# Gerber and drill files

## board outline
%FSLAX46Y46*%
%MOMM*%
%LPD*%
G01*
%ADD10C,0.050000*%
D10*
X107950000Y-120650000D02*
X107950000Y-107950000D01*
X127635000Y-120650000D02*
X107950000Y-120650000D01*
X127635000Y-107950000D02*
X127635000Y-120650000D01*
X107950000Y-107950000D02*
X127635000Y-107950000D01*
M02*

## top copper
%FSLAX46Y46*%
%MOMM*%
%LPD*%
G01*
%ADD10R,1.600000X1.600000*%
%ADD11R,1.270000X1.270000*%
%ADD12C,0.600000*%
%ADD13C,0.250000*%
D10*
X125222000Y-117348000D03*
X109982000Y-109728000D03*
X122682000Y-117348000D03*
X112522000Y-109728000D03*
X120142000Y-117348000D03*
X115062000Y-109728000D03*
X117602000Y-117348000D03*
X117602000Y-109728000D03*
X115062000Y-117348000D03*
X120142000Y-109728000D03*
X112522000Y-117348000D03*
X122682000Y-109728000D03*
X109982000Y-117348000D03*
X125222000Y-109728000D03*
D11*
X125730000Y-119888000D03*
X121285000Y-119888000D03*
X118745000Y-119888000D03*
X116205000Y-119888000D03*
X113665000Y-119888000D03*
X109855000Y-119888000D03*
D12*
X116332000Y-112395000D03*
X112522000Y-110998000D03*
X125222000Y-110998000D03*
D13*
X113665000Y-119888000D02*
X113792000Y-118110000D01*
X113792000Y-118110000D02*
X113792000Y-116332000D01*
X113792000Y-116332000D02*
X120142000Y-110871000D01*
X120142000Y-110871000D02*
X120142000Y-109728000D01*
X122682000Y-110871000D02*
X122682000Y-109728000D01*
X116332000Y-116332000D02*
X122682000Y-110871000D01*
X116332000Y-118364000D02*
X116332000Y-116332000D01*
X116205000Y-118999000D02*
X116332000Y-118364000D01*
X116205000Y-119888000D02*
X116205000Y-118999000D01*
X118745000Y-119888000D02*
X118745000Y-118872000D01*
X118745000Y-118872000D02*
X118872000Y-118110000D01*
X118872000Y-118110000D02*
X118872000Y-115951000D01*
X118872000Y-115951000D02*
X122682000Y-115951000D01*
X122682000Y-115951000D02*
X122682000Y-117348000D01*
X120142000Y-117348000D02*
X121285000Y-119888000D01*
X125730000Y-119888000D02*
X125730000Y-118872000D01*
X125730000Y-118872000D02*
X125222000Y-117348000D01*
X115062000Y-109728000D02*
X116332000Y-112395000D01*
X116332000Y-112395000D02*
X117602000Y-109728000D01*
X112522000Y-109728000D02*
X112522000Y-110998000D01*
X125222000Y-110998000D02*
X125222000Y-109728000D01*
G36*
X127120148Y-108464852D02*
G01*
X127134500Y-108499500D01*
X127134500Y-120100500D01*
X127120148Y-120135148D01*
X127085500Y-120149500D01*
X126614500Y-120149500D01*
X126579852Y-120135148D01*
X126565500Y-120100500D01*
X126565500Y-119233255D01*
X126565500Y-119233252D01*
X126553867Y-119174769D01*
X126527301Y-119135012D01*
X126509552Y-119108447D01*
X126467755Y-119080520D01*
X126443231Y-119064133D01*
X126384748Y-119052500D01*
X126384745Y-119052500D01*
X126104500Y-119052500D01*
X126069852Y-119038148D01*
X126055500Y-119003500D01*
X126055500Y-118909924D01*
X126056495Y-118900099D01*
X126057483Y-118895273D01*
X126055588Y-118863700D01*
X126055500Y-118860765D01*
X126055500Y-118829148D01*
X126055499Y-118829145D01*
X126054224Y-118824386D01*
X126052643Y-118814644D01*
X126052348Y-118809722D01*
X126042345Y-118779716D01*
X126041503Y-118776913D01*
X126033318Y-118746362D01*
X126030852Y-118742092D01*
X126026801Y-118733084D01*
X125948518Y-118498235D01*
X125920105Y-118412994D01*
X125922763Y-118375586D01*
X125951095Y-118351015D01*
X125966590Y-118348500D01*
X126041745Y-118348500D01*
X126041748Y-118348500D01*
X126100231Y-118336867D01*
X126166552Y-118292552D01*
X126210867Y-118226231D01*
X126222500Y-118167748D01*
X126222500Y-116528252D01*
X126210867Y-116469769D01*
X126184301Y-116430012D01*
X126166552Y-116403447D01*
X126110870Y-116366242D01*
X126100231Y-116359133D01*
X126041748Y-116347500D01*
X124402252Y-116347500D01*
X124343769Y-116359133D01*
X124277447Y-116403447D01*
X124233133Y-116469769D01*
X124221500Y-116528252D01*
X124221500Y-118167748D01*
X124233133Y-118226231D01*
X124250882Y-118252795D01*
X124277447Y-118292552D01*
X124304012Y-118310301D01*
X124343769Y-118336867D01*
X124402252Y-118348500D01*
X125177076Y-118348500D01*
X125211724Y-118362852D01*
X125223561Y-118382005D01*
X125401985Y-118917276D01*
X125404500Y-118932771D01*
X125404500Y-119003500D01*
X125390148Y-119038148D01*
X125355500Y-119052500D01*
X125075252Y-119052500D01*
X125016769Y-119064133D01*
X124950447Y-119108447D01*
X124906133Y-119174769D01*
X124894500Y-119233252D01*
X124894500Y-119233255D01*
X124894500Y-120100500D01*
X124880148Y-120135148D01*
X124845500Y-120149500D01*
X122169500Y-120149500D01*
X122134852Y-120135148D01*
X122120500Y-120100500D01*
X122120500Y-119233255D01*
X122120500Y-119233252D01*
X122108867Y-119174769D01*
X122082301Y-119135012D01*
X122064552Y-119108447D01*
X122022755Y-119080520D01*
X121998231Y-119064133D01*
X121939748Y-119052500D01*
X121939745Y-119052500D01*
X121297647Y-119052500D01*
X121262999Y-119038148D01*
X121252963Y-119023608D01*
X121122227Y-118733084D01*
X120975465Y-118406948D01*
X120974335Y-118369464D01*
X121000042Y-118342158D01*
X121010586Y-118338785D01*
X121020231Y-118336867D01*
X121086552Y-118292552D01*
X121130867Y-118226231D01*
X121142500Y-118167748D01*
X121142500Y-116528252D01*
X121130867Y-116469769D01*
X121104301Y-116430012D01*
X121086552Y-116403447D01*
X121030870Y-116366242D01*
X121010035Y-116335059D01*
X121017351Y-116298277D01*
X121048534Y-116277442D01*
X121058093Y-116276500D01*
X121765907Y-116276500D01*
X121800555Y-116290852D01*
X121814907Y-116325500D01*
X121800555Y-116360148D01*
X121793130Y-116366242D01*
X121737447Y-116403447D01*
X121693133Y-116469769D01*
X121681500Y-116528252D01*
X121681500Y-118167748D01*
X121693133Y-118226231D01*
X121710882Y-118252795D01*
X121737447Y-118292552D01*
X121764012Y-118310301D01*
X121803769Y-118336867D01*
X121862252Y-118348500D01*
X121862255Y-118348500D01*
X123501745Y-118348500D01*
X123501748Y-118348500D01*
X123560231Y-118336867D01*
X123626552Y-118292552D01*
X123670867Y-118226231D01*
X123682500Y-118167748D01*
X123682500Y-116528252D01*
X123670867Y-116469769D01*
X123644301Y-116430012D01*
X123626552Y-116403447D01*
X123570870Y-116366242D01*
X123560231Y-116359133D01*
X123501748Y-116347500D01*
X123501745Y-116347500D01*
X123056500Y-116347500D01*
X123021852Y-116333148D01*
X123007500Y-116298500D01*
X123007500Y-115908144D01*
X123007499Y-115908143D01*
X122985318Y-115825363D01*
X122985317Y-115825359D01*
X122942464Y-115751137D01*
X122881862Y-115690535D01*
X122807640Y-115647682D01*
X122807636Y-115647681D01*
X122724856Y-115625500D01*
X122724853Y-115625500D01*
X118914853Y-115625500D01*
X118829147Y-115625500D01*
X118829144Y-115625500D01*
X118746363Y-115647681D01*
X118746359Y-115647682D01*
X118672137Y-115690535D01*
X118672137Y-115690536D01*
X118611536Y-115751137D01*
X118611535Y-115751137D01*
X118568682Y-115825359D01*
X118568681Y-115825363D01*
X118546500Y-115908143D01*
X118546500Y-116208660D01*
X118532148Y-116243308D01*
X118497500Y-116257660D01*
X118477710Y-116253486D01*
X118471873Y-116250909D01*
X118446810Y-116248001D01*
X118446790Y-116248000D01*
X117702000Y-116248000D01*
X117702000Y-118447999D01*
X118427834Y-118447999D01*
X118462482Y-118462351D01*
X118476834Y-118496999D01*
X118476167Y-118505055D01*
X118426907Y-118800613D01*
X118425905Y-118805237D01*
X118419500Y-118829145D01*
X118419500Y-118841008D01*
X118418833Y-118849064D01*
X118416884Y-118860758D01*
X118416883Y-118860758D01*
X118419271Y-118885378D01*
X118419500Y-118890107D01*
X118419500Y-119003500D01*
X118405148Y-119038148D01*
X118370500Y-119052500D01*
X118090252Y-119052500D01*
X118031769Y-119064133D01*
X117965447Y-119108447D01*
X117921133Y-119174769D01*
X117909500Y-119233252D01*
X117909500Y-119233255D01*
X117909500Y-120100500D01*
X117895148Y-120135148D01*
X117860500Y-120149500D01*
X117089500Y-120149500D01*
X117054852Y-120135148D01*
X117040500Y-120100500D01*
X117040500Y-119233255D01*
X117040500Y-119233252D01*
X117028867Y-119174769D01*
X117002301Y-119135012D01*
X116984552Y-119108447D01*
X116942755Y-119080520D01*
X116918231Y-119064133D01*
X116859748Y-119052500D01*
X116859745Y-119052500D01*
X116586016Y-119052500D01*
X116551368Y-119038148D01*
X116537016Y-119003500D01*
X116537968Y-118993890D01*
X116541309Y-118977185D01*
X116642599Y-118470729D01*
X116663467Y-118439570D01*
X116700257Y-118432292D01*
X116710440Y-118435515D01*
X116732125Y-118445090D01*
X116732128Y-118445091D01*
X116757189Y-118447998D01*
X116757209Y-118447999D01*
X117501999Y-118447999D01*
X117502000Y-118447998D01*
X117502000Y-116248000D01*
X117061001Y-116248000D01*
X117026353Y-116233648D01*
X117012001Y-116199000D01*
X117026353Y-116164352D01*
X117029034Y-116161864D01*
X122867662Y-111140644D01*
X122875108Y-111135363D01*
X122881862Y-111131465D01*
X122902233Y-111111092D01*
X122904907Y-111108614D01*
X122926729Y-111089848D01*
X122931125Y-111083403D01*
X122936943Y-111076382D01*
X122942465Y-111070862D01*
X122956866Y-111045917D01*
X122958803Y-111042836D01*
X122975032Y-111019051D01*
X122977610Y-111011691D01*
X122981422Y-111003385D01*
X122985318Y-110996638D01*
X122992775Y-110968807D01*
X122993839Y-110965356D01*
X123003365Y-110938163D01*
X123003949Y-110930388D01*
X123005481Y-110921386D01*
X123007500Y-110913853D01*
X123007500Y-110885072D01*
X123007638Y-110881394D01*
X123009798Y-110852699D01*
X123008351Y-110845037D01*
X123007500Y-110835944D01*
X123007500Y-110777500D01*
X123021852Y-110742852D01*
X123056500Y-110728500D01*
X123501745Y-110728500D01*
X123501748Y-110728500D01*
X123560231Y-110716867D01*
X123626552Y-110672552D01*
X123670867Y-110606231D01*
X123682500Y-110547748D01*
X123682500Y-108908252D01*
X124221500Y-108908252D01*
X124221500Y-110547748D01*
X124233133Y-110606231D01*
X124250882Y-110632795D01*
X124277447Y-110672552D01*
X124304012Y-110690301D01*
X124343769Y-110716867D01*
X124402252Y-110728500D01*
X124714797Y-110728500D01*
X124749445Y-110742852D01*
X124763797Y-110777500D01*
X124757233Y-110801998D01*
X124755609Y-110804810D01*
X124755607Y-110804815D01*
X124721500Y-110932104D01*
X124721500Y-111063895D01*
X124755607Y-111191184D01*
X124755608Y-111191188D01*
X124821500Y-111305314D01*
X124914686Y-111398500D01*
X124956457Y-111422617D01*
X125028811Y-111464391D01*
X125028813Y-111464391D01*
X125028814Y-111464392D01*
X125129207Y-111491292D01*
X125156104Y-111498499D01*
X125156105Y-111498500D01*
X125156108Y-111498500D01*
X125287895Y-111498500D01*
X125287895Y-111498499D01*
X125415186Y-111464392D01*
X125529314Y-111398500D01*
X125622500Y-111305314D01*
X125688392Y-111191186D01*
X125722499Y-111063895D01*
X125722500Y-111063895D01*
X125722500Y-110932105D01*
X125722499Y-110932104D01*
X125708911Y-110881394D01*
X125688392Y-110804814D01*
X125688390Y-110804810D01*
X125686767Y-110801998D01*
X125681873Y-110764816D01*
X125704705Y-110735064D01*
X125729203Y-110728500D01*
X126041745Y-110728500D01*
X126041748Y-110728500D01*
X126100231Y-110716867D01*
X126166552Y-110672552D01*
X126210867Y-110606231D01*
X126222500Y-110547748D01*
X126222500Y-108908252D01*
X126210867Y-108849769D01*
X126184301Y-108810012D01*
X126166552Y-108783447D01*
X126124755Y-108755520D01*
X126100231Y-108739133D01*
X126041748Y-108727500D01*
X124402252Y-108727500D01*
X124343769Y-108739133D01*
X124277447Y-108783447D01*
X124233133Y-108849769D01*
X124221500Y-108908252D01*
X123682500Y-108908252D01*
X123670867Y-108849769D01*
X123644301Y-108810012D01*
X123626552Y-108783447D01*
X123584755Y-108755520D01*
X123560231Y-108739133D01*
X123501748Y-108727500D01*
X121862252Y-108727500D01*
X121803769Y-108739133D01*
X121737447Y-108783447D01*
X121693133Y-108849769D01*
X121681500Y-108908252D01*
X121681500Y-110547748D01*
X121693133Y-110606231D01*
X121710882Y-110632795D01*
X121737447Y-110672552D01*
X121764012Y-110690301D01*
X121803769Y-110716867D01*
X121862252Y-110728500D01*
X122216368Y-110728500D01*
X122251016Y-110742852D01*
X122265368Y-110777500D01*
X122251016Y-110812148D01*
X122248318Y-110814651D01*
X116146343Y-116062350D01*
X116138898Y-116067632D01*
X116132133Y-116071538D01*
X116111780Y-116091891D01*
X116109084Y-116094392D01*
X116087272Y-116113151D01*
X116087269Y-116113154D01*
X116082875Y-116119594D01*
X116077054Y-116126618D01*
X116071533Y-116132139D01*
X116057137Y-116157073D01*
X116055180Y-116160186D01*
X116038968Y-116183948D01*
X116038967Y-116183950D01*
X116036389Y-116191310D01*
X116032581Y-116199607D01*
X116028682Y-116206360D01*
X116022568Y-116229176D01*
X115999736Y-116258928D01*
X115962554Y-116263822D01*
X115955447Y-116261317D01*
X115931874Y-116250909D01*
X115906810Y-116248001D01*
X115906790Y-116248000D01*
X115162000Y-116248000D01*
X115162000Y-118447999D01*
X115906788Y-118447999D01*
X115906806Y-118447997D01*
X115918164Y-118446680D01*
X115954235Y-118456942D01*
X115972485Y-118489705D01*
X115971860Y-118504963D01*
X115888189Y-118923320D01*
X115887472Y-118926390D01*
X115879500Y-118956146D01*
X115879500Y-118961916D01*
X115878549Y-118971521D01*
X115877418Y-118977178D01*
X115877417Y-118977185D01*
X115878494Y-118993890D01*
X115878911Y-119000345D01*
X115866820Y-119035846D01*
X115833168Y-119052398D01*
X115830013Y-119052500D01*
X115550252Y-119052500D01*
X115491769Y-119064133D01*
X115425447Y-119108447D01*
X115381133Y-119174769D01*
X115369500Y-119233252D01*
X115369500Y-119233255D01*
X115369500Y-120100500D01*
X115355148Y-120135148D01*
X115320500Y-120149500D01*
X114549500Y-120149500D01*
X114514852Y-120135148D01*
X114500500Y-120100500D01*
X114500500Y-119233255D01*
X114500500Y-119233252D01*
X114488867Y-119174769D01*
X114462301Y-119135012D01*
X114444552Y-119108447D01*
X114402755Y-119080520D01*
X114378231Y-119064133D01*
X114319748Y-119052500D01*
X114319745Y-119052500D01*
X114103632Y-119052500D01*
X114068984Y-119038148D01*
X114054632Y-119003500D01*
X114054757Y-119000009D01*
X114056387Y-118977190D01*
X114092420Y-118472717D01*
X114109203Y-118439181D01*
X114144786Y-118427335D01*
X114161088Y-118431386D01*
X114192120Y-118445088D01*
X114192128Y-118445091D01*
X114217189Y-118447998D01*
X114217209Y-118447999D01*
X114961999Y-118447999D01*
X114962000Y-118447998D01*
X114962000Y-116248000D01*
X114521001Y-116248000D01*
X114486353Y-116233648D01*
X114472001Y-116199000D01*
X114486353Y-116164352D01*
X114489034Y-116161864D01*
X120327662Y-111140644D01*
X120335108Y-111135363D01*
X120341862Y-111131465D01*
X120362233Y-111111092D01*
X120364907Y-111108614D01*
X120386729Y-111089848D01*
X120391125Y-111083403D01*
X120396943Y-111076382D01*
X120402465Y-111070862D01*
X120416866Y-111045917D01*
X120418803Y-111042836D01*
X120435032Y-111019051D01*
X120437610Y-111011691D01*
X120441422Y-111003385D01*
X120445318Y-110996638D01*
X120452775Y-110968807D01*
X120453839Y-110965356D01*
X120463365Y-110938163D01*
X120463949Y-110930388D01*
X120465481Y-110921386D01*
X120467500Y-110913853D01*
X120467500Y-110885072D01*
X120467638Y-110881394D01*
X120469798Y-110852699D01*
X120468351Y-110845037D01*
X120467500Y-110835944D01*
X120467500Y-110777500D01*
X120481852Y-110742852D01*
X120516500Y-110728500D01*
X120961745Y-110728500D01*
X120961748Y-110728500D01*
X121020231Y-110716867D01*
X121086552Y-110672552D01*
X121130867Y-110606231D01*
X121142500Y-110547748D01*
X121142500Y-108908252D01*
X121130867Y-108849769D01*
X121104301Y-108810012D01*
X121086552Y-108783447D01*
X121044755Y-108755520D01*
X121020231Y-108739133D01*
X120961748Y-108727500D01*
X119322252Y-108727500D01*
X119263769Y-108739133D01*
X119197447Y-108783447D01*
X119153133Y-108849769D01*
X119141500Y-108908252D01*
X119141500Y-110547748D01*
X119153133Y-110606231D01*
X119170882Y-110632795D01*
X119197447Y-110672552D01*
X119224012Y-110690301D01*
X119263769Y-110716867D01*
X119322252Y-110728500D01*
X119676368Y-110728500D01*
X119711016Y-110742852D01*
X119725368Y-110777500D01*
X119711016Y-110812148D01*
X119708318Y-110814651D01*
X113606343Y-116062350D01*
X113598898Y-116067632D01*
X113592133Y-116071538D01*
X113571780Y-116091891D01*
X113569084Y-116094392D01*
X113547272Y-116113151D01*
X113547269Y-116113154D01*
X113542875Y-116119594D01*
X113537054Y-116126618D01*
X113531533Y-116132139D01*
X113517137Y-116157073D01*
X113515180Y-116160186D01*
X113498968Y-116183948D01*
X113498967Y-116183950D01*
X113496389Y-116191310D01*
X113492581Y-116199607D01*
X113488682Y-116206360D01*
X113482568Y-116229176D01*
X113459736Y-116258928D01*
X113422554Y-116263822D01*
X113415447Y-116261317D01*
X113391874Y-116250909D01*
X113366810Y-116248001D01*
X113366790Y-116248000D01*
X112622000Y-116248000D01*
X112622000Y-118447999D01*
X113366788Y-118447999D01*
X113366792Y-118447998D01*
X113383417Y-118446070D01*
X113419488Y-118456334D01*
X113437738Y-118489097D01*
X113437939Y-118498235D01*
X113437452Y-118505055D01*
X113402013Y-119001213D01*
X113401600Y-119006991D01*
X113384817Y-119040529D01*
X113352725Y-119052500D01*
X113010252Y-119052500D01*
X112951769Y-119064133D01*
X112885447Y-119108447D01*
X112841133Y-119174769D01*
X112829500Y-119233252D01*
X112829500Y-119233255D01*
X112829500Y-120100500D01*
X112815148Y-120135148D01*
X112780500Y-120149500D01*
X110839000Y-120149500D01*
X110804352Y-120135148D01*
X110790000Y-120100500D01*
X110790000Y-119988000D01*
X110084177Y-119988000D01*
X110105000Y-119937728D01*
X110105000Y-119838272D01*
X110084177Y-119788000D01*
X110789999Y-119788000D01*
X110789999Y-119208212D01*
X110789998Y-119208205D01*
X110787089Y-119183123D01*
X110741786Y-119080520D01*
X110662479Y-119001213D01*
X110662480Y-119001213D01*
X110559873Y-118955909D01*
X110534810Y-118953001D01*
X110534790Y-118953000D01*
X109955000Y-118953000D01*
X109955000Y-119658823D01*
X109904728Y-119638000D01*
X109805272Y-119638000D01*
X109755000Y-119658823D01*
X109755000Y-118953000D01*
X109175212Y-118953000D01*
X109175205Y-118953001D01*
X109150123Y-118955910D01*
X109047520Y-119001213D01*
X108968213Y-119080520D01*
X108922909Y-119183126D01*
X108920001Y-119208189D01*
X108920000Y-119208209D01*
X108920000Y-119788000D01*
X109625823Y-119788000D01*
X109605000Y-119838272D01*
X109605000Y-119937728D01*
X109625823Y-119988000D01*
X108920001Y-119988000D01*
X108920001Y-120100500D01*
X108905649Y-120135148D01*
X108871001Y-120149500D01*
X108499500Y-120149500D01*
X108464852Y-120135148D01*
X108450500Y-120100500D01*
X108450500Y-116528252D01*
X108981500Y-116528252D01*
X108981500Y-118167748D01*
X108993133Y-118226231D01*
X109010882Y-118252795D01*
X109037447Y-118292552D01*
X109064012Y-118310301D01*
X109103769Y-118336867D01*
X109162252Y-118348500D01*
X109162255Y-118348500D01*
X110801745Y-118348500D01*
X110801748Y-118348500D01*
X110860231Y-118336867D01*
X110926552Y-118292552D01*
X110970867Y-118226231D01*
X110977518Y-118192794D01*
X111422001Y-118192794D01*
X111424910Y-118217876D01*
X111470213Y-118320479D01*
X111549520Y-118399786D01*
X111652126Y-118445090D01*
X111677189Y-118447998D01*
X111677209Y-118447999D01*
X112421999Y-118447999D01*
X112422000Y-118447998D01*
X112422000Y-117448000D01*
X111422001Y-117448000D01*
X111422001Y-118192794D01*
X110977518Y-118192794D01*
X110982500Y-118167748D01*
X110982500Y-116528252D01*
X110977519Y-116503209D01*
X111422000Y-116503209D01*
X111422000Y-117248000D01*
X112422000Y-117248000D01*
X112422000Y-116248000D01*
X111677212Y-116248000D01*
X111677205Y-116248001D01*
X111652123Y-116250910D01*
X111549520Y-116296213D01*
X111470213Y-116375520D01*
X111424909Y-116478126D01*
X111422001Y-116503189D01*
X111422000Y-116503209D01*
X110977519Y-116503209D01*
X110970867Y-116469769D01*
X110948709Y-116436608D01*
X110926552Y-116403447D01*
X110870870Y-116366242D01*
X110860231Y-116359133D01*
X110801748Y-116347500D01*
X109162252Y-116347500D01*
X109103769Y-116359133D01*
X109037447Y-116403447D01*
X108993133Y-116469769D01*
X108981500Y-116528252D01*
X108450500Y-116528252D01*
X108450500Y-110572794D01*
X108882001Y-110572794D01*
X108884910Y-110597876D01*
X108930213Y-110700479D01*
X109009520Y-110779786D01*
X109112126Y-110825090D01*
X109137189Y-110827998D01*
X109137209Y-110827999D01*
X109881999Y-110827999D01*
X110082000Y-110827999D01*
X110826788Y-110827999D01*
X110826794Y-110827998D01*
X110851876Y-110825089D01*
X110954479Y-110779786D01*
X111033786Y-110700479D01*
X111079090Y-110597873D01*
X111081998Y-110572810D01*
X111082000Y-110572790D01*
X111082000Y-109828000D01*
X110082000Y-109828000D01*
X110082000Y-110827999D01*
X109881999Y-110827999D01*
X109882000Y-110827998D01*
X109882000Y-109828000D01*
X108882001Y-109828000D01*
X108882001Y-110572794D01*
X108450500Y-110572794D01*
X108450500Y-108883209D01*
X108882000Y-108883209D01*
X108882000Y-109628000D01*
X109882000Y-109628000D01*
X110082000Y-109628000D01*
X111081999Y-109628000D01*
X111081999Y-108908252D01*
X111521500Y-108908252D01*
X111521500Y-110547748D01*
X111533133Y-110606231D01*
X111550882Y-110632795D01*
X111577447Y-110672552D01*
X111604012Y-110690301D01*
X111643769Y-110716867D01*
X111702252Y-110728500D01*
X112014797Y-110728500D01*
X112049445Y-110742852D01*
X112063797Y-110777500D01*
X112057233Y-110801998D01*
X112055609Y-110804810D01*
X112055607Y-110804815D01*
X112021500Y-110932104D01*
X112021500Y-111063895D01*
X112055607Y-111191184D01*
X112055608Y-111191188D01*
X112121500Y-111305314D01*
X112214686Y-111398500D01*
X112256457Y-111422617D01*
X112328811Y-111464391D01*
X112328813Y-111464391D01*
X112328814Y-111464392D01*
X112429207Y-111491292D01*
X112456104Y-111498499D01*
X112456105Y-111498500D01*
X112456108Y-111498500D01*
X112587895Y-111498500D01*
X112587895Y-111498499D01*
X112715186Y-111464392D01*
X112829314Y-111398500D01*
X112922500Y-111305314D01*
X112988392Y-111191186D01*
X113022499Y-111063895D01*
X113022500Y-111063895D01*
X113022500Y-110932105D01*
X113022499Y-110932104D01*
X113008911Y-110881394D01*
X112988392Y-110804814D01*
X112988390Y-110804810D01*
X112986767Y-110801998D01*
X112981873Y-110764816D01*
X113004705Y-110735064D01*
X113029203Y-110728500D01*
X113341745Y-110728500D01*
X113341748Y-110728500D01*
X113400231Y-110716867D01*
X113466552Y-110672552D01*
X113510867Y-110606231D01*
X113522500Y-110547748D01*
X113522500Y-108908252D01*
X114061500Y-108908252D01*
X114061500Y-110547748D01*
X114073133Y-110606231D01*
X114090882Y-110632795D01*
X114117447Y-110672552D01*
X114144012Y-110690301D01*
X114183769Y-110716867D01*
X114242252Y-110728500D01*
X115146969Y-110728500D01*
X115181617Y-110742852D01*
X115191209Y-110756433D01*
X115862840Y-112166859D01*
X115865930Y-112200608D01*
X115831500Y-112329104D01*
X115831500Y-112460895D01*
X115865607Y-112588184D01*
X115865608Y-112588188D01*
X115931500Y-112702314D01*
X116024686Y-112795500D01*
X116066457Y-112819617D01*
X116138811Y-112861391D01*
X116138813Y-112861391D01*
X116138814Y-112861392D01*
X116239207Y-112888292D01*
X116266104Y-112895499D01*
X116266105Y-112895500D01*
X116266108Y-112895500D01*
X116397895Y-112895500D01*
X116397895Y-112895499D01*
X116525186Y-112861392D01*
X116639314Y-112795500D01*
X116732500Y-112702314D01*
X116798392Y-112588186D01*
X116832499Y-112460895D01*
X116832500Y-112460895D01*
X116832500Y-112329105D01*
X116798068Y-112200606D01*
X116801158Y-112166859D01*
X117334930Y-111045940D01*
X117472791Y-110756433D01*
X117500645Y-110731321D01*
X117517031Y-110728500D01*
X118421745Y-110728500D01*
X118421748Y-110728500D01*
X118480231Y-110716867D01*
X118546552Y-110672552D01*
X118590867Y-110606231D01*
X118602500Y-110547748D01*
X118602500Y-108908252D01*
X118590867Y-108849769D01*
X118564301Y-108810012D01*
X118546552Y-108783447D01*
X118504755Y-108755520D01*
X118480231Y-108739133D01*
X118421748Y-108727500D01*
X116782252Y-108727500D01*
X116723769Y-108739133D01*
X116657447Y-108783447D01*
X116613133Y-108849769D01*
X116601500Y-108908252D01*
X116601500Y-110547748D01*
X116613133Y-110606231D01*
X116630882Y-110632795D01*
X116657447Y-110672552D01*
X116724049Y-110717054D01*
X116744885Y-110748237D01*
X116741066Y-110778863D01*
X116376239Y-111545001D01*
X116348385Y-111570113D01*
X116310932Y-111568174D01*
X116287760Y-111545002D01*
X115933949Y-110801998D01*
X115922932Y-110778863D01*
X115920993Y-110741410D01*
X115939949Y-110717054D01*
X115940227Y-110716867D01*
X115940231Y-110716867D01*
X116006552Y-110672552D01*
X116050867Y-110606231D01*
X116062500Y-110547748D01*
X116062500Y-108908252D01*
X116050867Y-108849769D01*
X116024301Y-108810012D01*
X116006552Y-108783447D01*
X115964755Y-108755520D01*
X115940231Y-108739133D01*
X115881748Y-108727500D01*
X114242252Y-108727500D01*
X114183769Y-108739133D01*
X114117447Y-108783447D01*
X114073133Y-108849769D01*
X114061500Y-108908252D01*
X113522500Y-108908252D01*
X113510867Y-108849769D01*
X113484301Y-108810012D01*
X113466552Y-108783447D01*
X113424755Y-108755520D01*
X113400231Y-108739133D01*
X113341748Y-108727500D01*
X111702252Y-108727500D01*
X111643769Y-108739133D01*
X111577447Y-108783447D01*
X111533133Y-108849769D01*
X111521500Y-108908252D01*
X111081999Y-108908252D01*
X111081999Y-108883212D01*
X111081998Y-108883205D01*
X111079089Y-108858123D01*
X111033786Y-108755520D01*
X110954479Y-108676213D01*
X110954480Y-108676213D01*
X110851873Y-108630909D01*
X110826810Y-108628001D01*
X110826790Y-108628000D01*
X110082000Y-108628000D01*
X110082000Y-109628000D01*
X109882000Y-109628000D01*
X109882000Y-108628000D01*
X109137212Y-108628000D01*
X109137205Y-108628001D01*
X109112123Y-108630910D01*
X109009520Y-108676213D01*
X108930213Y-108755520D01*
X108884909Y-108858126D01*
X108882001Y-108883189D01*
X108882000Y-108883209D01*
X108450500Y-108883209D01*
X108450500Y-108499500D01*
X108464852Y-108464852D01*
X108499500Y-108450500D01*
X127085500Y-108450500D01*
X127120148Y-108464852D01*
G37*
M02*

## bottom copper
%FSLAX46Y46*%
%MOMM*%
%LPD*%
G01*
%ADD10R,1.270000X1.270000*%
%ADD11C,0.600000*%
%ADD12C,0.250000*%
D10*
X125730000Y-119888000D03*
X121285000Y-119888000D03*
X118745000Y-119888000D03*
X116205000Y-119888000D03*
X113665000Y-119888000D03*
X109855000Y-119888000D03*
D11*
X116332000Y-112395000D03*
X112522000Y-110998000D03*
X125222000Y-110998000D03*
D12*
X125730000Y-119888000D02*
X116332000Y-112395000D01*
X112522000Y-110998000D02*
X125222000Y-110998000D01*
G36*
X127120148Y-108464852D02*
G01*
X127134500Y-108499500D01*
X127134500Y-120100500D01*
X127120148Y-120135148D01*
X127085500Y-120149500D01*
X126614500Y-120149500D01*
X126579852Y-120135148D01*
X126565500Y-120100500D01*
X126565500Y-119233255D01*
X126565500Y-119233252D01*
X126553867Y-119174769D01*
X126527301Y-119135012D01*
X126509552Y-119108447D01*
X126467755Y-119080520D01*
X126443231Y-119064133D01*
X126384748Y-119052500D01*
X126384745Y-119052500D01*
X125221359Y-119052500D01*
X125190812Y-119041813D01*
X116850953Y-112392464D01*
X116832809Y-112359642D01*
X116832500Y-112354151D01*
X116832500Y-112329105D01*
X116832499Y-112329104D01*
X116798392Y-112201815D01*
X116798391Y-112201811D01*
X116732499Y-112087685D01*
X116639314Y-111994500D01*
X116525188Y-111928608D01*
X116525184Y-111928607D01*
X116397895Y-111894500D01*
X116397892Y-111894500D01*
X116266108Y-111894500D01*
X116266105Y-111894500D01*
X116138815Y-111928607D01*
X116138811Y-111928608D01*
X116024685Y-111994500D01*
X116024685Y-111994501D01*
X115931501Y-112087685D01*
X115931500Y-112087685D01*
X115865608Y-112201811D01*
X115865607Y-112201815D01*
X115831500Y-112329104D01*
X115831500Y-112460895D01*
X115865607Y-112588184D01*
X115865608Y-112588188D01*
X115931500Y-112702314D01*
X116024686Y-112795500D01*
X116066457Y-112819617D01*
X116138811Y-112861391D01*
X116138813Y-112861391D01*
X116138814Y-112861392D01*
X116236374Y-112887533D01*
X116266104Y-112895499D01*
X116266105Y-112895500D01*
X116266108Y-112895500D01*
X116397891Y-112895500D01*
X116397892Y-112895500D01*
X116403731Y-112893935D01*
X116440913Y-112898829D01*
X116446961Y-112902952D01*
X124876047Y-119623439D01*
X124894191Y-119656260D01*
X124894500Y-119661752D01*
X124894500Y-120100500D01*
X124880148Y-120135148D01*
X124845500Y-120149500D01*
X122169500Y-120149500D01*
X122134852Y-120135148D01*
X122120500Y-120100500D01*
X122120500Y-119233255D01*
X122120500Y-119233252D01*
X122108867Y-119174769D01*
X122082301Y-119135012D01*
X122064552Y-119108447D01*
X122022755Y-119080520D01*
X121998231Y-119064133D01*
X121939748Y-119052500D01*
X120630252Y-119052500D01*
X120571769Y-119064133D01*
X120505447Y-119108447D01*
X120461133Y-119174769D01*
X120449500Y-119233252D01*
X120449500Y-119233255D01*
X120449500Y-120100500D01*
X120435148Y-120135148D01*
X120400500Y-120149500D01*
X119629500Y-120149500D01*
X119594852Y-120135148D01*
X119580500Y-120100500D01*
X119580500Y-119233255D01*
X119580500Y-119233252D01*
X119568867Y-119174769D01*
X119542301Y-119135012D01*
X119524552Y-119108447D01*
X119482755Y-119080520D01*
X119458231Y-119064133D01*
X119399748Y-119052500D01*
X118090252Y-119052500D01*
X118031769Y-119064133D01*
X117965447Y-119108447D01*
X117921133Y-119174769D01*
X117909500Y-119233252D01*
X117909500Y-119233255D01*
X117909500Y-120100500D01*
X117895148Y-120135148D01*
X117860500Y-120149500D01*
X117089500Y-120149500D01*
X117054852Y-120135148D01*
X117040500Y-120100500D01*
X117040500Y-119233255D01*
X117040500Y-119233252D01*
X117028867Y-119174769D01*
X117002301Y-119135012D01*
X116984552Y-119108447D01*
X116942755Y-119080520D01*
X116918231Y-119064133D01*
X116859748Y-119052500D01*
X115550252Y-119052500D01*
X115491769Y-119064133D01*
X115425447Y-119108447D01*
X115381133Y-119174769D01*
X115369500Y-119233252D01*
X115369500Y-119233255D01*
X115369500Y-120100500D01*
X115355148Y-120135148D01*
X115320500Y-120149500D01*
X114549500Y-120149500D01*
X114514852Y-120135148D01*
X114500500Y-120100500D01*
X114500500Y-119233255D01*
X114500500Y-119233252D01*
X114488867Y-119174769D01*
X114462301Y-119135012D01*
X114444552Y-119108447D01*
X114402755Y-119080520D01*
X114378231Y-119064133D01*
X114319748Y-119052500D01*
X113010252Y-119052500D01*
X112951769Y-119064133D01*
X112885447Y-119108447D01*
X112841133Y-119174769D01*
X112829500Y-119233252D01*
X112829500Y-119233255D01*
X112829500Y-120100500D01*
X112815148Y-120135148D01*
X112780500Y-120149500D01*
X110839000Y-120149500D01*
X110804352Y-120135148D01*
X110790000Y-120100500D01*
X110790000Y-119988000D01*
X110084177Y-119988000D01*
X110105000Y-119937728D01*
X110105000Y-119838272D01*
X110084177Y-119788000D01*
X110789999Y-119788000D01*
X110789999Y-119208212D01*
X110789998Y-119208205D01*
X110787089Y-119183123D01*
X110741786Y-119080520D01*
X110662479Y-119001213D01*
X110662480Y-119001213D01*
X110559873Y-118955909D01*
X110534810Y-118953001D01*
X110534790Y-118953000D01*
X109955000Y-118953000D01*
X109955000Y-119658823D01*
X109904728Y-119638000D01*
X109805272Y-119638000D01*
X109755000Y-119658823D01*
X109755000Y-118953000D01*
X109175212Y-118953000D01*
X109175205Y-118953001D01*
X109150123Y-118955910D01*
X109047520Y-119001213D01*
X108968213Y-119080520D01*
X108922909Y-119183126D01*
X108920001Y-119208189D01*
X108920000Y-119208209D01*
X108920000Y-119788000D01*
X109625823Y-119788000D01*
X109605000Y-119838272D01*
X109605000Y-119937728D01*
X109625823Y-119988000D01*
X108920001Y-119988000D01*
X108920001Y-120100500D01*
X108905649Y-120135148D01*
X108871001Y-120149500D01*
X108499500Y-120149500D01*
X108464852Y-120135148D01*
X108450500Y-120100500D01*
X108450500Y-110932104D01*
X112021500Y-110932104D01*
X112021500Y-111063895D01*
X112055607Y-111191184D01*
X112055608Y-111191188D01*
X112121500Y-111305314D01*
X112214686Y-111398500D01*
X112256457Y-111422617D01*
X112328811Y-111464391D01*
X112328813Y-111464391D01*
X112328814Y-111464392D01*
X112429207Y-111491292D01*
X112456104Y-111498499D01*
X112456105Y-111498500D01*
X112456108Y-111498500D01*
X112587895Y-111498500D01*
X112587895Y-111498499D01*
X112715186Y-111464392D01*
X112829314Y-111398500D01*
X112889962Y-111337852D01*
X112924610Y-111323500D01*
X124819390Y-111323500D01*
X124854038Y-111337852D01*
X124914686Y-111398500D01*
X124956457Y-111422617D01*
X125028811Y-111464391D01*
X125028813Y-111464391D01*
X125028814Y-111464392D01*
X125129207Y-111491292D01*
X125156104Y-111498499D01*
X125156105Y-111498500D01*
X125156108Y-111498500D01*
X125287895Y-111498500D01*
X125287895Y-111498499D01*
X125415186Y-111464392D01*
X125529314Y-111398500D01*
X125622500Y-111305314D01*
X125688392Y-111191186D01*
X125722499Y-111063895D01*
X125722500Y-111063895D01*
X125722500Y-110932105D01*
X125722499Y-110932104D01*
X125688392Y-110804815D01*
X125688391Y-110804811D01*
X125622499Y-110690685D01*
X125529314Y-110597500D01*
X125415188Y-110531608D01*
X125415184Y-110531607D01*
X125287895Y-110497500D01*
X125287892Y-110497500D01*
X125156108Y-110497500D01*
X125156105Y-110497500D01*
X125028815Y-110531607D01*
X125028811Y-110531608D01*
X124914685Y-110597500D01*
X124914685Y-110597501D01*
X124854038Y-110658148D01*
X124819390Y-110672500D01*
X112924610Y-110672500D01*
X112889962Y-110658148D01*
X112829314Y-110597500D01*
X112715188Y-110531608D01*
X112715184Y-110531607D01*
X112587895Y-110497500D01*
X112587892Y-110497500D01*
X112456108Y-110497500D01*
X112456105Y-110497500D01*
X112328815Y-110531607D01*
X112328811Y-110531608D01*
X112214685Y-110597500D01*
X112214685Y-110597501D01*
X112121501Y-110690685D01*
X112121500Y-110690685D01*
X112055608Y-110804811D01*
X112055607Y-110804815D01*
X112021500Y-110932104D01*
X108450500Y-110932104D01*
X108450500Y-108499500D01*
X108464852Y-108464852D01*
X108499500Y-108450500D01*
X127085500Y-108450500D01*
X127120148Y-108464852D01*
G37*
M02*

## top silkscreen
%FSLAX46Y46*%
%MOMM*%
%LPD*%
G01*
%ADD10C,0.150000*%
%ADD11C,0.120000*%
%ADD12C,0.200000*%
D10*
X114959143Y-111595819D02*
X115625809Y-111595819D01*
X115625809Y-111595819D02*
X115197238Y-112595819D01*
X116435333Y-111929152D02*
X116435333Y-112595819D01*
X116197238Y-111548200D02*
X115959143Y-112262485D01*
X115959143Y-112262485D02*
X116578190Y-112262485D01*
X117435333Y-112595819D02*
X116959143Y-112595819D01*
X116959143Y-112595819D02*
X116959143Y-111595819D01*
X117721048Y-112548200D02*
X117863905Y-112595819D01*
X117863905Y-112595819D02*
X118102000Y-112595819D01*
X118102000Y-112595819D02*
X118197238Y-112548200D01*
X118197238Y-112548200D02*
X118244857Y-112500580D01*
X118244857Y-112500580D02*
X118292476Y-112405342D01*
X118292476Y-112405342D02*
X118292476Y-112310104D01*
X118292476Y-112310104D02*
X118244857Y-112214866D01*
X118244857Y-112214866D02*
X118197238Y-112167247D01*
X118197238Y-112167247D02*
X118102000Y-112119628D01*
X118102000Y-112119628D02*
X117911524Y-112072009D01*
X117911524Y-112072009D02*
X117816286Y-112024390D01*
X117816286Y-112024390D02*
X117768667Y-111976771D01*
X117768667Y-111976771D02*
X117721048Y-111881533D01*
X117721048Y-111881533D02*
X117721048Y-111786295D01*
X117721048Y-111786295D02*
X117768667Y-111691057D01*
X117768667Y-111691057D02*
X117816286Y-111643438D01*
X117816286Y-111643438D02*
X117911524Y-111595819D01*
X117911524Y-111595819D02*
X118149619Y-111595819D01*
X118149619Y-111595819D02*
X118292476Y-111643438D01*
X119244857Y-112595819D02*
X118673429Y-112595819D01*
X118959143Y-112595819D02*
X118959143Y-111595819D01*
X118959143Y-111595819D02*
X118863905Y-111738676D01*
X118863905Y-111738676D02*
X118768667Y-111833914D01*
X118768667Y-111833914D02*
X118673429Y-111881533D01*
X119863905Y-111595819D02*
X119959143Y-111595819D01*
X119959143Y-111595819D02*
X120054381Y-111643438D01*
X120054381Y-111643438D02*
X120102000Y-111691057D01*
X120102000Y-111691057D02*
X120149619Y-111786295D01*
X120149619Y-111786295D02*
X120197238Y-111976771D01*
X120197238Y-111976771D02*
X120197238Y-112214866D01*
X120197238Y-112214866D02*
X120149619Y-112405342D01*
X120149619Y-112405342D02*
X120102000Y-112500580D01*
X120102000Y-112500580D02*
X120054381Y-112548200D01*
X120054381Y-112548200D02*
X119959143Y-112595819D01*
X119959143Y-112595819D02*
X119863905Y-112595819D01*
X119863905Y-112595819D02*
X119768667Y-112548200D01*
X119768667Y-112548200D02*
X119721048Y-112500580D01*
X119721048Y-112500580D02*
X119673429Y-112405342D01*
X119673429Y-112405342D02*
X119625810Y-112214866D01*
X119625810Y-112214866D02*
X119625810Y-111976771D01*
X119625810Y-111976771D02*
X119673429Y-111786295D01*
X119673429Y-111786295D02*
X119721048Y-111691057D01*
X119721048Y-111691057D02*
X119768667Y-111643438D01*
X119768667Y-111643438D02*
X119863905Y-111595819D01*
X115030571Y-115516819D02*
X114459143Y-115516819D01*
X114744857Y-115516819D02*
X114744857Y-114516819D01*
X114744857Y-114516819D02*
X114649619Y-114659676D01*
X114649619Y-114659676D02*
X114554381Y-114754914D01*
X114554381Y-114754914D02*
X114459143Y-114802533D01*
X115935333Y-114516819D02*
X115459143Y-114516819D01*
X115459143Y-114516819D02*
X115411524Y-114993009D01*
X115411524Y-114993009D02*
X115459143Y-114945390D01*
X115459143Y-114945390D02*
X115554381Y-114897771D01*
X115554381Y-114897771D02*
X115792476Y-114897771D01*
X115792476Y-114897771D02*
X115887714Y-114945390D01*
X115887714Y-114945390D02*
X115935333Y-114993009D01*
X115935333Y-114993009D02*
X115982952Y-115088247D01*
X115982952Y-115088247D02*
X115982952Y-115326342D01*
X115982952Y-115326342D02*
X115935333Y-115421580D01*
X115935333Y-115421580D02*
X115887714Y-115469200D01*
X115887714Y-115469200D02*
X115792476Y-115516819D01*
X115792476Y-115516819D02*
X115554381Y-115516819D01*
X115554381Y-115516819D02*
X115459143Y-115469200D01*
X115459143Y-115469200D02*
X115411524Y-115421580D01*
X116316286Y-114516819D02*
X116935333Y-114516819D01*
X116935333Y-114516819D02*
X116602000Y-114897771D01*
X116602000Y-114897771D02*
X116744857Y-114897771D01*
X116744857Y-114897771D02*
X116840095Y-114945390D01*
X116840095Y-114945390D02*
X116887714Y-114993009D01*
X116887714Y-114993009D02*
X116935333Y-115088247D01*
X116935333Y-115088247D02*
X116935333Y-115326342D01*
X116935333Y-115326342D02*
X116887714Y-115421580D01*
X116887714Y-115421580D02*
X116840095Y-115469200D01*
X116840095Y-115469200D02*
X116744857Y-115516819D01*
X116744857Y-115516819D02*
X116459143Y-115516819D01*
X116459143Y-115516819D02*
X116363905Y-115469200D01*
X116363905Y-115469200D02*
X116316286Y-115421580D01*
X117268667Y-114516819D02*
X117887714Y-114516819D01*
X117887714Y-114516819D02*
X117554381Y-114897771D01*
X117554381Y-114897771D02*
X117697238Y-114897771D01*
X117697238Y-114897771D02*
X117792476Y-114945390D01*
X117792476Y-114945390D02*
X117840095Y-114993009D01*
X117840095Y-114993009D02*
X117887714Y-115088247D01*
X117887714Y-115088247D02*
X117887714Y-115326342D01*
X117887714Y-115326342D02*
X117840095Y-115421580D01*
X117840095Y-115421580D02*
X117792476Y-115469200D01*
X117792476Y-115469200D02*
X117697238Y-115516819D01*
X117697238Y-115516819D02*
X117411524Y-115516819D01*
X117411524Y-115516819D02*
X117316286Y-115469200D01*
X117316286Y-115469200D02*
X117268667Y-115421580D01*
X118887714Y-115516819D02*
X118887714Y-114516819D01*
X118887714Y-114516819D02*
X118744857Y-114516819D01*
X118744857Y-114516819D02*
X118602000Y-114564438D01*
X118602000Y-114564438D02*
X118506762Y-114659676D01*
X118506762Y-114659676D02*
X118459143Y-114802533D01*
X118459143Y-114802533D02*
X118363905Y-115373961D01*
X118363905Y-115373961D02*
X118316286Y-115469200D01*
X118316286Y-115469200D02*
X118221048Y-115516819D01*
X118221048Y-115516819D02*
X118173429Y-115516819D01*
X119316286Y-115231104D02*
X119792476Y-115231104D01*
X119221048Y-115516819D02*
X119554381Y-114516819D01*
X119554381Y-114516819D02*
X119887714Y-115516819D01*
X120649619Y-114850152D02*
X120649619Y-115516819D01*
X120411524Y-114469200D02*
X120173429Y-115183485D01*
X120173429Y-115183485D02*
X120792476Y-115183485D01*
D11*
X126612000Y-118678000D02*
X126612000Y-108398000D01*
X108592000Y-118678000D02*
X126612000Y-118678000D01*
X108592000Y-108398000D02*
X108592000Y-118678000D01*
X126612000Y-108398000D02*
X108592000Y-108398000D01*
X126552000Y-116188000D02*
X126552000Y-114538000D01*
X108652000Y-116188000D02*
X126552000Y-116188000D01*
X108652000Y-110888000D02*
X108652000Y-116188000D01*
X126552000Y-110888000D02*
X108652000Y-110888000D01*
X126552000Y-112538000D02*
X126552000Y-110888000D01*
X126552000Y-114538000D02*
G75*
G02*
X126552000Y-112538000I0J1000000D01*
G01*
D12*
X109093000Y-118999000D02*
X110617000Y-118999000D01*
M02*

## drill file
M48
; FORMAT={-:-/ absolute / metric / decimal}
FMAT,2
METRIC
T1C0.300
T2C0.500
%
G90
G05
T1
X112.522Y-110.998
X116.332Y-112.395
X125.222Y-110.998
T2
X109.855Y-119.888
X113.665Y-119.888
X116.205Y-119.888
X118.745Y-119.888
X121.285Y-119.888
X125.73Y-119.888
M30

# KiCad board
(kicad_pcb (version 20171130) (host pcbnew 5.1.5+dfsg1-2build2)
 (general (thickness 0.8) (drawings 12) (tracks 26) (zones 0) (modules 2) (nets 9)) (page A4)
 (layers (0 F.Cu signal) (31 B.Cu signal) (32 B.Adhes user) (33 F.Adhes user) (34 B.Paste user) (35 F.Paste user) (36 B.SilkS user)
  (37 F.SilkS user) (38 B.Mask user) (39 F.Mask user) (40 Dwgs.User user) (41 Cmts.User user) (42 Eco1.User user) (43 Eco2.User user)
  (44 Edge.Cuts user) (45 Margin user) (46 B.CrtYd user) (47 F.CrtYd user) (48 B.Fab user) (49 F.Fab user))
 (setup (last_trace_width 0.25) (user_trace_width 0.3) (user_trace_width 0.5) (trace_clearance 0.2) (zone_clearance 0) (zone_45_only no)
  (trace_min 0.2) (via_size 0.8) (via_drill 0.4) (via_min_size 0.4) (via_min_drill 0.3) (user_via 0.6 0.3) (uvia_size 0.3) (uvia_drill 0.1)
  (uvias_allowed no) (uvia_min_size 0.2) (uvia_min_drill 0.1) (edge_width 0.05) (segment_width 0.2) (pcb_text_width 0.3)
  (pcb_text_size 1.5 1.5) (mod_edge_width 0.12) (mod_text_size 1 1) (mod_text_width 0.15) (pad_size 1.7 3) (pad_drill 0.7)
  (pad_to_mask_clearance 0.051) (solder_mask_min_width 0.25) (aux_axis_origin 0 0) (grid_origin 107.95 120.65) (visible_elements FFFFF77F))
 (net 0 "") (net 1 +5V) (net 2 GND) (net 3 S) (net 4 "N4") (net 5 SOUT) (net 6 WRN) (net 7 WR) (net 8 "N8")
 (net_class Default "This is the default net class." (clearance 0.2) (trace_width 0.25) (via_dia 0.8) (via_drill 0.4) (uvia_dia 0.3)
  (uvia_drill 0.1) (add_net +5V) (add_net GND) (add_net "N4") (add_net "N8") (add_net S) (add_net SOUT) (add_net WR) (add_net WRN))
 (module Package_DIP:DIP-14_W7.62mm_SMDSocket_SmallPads (layer F.Cu) (at 117.602 113.538 270)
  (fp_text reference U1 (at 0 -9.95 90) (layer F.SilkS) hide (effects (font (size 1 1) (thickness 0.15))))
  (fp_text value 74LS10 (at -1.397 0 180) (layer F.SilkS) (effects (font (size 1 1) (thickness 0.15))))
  (fp_line (start 5.14 -9.01) (end -5.14 -9.01) (layer F.SilkS) (width 0.12))
  (fp_line (start 5.14 9.01) (end 5.14 -9.01) (layer F.SilkS) (width 0.12))
  (fp_line (start -5.14 9.01) (end 5.14 9.01) (layer F.SilkS) (width 0.12))
  (fp_line (start -5.14 -9.01) (end -5.14 9.01) (layer F.SilkS) (width 0.12))
  (fp_line (start 2.65 -8.95) (end 1 -8.95) (layer F.SilkS) (width 0.12))
  (fp_line (start 2.65 8.95) (end 2.65 -8.95) (layer F.SilkS) (width 0.12))
  (fp_line (start -2.65 8.95) (end 2.65 8.95) (layer F.SilkS) (width 0.12))
  (fp_line (start -2.65 -8.95) (end -2.65 8.95) (layer F.SilkS) (width 0.12))
  (fp_line (start -1 -8.95) (end -2.65 -8.95) (layer F.SilkS) (width 0.12))
  (fp_arc (start 0 -8.95) (end -1 -8.95) (angle -180) (layer F.SilkS) (width 0.12))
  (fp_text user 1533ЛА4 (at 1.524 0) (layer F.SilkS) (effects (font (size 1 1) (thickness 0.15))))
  (pad 14 smd rect (at 3.81 -7.62 270) (size 1.6 1.6) (layers F.Cu F.Paste F.Mask) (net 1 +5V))
  (pad 7 smd rect (at -3.81 7.62 270) (size 1.6 1.6) (layers F.Cu F.Paste F.Mask) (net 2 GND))
  (pad 13 smd rect (at 3.81 -5.08 270) (size 1.6 1.6) (layers F.Cu F.Paste F.Mask) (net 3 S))
  (pad 6 smd rect (at -3.81 5.08 270) (size 1.6 1.6) (layers F.Cu F.Paste F.Mask) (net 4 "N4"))
  (pad 12 smd rect (at 3.81 -2.54 270) (size 1.6 1.6) (layers F.Cu F.Paste F.Mask) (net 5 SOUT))
  (pad 5 smd rect (at -3.81 2.54 270) (size 1.6 1.6) (layers F.Cu F.Paste F.Mask) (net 1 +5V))
  (pad 11 smd rect (at 3.81 0 270) (size 1.6 1.6) (layers F.Cu F.Paste F.Mask) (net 2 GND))
  (pad 4 smd rect (at -3.81 0 270) (size 1.6 1.6) (layers F.Cu F.Paste F.Mask) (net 1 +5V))
  (pad 10 smd rect (at 3.81 2.54 270) (size 1.6 1.6) (layers F.Cu F.Paste F.Mask) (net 2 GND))
  (pad 3 smd rect (at -3.81 -2.54 270) (size 1.6 1.6) (layers F.Cu F.Paste F.Mask) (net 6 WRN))
  (pad 9 smd rect (at 3.81 5.08 270) (size 1.6 1.6) (layers F.Cu F.Paste F.Mask) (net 2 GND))
  (pad 2 smd rect (at -3.81 -5.08 270) (size 1.6 1.6) (layers F.Cu F.Paste F.Mask) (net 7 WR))
  (pad 8 smd rect (at 3.81 7.62 270) (size 1.6 1.6) (layers F.Cu F.Paste F.Mask) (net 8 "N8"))
  (pad 1 smd rect (at -3.81 -7.62 270) (size 1.6 1.6) (layers F.Cu F.Paste F.Mask) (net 4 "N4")))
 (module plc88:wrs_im (layer F.Cu) (at 115.57 117.348)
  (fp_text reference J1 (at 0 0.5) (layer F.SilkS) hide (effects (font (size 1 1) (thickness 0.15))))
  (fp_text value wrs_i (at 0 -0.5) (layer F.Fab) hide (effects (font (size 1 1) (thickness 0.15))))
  (fp_line (start -6.477 1.651) (end -4.953 1.651) (layer F.SilkS) (width 0.2))
  (pad 6 thru_hole rect (at 10.16 2.54) (size 1.27 1.27) (drill 0.5) (layers *.Cu *.Mask) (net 1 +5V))
  (pad 5 thru_hole rect (at 5.715 2.54) (size 1.27 1.27) (drill 0.5) (layers *.Cu *.Mask) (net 5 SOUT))
  (pad 4 thru_hole rect (at 3.175 2.54) (size 1.27 1.27) (drill 0.5) (layers *.Cu *.Mask) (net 3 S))
  (pad 3 thru_hole rect (at 0.635 2.54) (size 1.27 1.27) (drill 0.5) (layers *.Cu *.Mask) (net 7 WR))
  (pad 2 thru_hole rect (at -1.905 2.54) (size 1.27 1.27) (drill 0.5) (layers *.Cu *.Mask) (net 6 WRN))
  (pad 1 thru_hole rect (at -5.715 2.54) (size 1.27 1.27) (drill 0.5) (layers *.Cu *.Mask) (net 2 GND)))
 (gr_line (start 107.95 120.65) (end 107.95 107.95) (layer Edge.Cuts) (width 0.05))
 (gr_line (start 127.635 120.65) (end 107.95 120.65) (layer Edge.Cuts) (width 0.05))
 (gr_line (start 127.635 107.95) (end 127.635 120.65) (layer Edge.Cuts) (width 0.05))
 (gr_line (start 107.95 107.95) (end 127.635 107.95) (layer Edge.Cuts) (width 0.05))
 (segment (start 113.665 119.888) (end 113.792 118.11) (width 0.25) (layer F.Cu) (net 6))
 (segment (start 113.792 118.11) (end 113.792 116.332) (width 0.25) (layer F.Cu) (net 6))
 (segment (start 113.792 116.332) (end 120.142 110.871) (width 0.25) (layer F.Cu) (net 6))
 (segment (start 120.142 110.871) (end 120.142 109.728) (width 0.25) (layer F.Cu) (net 6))
 (segment (start 122.682 110.871) (end 122.682 109.728) (width 0.25) (layer F.Cu) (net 7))
 (segment (start 116.332 116.332) (end 122.682 110.871) (width 0.25) (layer F.Cu) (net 7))
 (segment (start 116.332 118.364) (end 116.332 116.332) (width 0.25) (layer F.Cu) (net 7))
 (segment (start 116.205 118.999) (end 116.332 118.364) (width 0.25) (layer F.Cu) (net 7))
 (segment (start 116.205 119.888) (end 116.205 118.999) (width 0.25) (layer F.Cu) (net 7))
 (segment (start 118.745 119.888) (end 118.745 118.872) (width 0.25) (layer F.Cu) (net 3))
 (segment (start 118.745 118.872) (end 118.872 118.11) (width 0.25) (layer F.Cu) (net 3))
 (segment (start 118.872 118.11) (end 118.872 115.951) (width 0.25) (layer F.Cu) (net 3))
 (segment (start 118.872 115.951) (end 122.682 115.951) (width 0.25) (layer F.Cu) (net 3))
 (segment (start 122.682 115.951) (end 122.682 117.348) (width 0.25) (layer F.Cu) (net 3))
 (segment (start 120.142 117.348) (end 121.285 119.888) (width 0.25) (layer F.Cu) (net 5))
 (segment (start 125.73 119.888) (end 125.73 118.872) (width 0.25) (layer F.Cu) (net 1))
 (segment (start 125.73 118.872) (end 125.222 117.348) (width 0.25) (layer F.Cu) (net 1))
 (segment (start 125.73 119.888) (end 116.332 112.395) (width 0.25) (layer B.Cu) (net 1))
 (segment (start 115.062 109.728) (end 116.332 112.395) (width 0.25) (layer F.Cu) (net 1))
 (segment (start 116.332 112.395) (end 117.602 109.728) (width 0.25) (layer F.Cu) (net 1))
 (via (at 116.332 112.395) (size 0.6) (drill 0.3) (layers F.Cu B.Cu) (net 1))
 (segment (start 112.522 109.728) (end 112.522 110.998) (width 0.25) (layer F.Cu) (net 4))
 (via (at 112.522 110.998) (size 0.6) (drill 0.3) (layers F.Cu B.Cu) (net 4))
 (segment (start 112.522 110.998) (end 125.222 110.998) (width 0.25) (layer B.Cu) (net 4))
 (segment (start 125.222 110.998) (end 125.222 109.728) (width 0.25) (layer F.Cu) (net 4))
 (via (at 125.222 110.998) (size 0.6) (drill 0.3) (layers F.Cu B.Cu) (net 4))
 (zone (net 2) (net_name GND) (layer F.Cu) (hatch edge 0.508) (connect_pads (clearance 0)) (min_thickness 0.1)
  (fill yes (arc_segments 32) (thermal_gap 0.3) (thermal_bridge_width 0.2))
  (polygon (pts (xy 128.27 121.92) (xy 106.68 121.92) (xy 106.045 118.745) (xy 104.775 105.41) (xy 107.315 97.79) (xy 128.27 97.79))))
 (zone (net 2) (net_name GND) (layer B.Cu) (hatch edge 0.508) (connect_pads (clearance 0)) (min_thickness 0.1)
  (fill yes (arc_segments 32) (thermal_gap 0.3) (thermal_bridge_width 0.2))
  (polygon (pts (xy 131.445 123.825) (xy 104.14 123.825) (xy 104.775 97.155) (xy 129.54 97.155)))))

